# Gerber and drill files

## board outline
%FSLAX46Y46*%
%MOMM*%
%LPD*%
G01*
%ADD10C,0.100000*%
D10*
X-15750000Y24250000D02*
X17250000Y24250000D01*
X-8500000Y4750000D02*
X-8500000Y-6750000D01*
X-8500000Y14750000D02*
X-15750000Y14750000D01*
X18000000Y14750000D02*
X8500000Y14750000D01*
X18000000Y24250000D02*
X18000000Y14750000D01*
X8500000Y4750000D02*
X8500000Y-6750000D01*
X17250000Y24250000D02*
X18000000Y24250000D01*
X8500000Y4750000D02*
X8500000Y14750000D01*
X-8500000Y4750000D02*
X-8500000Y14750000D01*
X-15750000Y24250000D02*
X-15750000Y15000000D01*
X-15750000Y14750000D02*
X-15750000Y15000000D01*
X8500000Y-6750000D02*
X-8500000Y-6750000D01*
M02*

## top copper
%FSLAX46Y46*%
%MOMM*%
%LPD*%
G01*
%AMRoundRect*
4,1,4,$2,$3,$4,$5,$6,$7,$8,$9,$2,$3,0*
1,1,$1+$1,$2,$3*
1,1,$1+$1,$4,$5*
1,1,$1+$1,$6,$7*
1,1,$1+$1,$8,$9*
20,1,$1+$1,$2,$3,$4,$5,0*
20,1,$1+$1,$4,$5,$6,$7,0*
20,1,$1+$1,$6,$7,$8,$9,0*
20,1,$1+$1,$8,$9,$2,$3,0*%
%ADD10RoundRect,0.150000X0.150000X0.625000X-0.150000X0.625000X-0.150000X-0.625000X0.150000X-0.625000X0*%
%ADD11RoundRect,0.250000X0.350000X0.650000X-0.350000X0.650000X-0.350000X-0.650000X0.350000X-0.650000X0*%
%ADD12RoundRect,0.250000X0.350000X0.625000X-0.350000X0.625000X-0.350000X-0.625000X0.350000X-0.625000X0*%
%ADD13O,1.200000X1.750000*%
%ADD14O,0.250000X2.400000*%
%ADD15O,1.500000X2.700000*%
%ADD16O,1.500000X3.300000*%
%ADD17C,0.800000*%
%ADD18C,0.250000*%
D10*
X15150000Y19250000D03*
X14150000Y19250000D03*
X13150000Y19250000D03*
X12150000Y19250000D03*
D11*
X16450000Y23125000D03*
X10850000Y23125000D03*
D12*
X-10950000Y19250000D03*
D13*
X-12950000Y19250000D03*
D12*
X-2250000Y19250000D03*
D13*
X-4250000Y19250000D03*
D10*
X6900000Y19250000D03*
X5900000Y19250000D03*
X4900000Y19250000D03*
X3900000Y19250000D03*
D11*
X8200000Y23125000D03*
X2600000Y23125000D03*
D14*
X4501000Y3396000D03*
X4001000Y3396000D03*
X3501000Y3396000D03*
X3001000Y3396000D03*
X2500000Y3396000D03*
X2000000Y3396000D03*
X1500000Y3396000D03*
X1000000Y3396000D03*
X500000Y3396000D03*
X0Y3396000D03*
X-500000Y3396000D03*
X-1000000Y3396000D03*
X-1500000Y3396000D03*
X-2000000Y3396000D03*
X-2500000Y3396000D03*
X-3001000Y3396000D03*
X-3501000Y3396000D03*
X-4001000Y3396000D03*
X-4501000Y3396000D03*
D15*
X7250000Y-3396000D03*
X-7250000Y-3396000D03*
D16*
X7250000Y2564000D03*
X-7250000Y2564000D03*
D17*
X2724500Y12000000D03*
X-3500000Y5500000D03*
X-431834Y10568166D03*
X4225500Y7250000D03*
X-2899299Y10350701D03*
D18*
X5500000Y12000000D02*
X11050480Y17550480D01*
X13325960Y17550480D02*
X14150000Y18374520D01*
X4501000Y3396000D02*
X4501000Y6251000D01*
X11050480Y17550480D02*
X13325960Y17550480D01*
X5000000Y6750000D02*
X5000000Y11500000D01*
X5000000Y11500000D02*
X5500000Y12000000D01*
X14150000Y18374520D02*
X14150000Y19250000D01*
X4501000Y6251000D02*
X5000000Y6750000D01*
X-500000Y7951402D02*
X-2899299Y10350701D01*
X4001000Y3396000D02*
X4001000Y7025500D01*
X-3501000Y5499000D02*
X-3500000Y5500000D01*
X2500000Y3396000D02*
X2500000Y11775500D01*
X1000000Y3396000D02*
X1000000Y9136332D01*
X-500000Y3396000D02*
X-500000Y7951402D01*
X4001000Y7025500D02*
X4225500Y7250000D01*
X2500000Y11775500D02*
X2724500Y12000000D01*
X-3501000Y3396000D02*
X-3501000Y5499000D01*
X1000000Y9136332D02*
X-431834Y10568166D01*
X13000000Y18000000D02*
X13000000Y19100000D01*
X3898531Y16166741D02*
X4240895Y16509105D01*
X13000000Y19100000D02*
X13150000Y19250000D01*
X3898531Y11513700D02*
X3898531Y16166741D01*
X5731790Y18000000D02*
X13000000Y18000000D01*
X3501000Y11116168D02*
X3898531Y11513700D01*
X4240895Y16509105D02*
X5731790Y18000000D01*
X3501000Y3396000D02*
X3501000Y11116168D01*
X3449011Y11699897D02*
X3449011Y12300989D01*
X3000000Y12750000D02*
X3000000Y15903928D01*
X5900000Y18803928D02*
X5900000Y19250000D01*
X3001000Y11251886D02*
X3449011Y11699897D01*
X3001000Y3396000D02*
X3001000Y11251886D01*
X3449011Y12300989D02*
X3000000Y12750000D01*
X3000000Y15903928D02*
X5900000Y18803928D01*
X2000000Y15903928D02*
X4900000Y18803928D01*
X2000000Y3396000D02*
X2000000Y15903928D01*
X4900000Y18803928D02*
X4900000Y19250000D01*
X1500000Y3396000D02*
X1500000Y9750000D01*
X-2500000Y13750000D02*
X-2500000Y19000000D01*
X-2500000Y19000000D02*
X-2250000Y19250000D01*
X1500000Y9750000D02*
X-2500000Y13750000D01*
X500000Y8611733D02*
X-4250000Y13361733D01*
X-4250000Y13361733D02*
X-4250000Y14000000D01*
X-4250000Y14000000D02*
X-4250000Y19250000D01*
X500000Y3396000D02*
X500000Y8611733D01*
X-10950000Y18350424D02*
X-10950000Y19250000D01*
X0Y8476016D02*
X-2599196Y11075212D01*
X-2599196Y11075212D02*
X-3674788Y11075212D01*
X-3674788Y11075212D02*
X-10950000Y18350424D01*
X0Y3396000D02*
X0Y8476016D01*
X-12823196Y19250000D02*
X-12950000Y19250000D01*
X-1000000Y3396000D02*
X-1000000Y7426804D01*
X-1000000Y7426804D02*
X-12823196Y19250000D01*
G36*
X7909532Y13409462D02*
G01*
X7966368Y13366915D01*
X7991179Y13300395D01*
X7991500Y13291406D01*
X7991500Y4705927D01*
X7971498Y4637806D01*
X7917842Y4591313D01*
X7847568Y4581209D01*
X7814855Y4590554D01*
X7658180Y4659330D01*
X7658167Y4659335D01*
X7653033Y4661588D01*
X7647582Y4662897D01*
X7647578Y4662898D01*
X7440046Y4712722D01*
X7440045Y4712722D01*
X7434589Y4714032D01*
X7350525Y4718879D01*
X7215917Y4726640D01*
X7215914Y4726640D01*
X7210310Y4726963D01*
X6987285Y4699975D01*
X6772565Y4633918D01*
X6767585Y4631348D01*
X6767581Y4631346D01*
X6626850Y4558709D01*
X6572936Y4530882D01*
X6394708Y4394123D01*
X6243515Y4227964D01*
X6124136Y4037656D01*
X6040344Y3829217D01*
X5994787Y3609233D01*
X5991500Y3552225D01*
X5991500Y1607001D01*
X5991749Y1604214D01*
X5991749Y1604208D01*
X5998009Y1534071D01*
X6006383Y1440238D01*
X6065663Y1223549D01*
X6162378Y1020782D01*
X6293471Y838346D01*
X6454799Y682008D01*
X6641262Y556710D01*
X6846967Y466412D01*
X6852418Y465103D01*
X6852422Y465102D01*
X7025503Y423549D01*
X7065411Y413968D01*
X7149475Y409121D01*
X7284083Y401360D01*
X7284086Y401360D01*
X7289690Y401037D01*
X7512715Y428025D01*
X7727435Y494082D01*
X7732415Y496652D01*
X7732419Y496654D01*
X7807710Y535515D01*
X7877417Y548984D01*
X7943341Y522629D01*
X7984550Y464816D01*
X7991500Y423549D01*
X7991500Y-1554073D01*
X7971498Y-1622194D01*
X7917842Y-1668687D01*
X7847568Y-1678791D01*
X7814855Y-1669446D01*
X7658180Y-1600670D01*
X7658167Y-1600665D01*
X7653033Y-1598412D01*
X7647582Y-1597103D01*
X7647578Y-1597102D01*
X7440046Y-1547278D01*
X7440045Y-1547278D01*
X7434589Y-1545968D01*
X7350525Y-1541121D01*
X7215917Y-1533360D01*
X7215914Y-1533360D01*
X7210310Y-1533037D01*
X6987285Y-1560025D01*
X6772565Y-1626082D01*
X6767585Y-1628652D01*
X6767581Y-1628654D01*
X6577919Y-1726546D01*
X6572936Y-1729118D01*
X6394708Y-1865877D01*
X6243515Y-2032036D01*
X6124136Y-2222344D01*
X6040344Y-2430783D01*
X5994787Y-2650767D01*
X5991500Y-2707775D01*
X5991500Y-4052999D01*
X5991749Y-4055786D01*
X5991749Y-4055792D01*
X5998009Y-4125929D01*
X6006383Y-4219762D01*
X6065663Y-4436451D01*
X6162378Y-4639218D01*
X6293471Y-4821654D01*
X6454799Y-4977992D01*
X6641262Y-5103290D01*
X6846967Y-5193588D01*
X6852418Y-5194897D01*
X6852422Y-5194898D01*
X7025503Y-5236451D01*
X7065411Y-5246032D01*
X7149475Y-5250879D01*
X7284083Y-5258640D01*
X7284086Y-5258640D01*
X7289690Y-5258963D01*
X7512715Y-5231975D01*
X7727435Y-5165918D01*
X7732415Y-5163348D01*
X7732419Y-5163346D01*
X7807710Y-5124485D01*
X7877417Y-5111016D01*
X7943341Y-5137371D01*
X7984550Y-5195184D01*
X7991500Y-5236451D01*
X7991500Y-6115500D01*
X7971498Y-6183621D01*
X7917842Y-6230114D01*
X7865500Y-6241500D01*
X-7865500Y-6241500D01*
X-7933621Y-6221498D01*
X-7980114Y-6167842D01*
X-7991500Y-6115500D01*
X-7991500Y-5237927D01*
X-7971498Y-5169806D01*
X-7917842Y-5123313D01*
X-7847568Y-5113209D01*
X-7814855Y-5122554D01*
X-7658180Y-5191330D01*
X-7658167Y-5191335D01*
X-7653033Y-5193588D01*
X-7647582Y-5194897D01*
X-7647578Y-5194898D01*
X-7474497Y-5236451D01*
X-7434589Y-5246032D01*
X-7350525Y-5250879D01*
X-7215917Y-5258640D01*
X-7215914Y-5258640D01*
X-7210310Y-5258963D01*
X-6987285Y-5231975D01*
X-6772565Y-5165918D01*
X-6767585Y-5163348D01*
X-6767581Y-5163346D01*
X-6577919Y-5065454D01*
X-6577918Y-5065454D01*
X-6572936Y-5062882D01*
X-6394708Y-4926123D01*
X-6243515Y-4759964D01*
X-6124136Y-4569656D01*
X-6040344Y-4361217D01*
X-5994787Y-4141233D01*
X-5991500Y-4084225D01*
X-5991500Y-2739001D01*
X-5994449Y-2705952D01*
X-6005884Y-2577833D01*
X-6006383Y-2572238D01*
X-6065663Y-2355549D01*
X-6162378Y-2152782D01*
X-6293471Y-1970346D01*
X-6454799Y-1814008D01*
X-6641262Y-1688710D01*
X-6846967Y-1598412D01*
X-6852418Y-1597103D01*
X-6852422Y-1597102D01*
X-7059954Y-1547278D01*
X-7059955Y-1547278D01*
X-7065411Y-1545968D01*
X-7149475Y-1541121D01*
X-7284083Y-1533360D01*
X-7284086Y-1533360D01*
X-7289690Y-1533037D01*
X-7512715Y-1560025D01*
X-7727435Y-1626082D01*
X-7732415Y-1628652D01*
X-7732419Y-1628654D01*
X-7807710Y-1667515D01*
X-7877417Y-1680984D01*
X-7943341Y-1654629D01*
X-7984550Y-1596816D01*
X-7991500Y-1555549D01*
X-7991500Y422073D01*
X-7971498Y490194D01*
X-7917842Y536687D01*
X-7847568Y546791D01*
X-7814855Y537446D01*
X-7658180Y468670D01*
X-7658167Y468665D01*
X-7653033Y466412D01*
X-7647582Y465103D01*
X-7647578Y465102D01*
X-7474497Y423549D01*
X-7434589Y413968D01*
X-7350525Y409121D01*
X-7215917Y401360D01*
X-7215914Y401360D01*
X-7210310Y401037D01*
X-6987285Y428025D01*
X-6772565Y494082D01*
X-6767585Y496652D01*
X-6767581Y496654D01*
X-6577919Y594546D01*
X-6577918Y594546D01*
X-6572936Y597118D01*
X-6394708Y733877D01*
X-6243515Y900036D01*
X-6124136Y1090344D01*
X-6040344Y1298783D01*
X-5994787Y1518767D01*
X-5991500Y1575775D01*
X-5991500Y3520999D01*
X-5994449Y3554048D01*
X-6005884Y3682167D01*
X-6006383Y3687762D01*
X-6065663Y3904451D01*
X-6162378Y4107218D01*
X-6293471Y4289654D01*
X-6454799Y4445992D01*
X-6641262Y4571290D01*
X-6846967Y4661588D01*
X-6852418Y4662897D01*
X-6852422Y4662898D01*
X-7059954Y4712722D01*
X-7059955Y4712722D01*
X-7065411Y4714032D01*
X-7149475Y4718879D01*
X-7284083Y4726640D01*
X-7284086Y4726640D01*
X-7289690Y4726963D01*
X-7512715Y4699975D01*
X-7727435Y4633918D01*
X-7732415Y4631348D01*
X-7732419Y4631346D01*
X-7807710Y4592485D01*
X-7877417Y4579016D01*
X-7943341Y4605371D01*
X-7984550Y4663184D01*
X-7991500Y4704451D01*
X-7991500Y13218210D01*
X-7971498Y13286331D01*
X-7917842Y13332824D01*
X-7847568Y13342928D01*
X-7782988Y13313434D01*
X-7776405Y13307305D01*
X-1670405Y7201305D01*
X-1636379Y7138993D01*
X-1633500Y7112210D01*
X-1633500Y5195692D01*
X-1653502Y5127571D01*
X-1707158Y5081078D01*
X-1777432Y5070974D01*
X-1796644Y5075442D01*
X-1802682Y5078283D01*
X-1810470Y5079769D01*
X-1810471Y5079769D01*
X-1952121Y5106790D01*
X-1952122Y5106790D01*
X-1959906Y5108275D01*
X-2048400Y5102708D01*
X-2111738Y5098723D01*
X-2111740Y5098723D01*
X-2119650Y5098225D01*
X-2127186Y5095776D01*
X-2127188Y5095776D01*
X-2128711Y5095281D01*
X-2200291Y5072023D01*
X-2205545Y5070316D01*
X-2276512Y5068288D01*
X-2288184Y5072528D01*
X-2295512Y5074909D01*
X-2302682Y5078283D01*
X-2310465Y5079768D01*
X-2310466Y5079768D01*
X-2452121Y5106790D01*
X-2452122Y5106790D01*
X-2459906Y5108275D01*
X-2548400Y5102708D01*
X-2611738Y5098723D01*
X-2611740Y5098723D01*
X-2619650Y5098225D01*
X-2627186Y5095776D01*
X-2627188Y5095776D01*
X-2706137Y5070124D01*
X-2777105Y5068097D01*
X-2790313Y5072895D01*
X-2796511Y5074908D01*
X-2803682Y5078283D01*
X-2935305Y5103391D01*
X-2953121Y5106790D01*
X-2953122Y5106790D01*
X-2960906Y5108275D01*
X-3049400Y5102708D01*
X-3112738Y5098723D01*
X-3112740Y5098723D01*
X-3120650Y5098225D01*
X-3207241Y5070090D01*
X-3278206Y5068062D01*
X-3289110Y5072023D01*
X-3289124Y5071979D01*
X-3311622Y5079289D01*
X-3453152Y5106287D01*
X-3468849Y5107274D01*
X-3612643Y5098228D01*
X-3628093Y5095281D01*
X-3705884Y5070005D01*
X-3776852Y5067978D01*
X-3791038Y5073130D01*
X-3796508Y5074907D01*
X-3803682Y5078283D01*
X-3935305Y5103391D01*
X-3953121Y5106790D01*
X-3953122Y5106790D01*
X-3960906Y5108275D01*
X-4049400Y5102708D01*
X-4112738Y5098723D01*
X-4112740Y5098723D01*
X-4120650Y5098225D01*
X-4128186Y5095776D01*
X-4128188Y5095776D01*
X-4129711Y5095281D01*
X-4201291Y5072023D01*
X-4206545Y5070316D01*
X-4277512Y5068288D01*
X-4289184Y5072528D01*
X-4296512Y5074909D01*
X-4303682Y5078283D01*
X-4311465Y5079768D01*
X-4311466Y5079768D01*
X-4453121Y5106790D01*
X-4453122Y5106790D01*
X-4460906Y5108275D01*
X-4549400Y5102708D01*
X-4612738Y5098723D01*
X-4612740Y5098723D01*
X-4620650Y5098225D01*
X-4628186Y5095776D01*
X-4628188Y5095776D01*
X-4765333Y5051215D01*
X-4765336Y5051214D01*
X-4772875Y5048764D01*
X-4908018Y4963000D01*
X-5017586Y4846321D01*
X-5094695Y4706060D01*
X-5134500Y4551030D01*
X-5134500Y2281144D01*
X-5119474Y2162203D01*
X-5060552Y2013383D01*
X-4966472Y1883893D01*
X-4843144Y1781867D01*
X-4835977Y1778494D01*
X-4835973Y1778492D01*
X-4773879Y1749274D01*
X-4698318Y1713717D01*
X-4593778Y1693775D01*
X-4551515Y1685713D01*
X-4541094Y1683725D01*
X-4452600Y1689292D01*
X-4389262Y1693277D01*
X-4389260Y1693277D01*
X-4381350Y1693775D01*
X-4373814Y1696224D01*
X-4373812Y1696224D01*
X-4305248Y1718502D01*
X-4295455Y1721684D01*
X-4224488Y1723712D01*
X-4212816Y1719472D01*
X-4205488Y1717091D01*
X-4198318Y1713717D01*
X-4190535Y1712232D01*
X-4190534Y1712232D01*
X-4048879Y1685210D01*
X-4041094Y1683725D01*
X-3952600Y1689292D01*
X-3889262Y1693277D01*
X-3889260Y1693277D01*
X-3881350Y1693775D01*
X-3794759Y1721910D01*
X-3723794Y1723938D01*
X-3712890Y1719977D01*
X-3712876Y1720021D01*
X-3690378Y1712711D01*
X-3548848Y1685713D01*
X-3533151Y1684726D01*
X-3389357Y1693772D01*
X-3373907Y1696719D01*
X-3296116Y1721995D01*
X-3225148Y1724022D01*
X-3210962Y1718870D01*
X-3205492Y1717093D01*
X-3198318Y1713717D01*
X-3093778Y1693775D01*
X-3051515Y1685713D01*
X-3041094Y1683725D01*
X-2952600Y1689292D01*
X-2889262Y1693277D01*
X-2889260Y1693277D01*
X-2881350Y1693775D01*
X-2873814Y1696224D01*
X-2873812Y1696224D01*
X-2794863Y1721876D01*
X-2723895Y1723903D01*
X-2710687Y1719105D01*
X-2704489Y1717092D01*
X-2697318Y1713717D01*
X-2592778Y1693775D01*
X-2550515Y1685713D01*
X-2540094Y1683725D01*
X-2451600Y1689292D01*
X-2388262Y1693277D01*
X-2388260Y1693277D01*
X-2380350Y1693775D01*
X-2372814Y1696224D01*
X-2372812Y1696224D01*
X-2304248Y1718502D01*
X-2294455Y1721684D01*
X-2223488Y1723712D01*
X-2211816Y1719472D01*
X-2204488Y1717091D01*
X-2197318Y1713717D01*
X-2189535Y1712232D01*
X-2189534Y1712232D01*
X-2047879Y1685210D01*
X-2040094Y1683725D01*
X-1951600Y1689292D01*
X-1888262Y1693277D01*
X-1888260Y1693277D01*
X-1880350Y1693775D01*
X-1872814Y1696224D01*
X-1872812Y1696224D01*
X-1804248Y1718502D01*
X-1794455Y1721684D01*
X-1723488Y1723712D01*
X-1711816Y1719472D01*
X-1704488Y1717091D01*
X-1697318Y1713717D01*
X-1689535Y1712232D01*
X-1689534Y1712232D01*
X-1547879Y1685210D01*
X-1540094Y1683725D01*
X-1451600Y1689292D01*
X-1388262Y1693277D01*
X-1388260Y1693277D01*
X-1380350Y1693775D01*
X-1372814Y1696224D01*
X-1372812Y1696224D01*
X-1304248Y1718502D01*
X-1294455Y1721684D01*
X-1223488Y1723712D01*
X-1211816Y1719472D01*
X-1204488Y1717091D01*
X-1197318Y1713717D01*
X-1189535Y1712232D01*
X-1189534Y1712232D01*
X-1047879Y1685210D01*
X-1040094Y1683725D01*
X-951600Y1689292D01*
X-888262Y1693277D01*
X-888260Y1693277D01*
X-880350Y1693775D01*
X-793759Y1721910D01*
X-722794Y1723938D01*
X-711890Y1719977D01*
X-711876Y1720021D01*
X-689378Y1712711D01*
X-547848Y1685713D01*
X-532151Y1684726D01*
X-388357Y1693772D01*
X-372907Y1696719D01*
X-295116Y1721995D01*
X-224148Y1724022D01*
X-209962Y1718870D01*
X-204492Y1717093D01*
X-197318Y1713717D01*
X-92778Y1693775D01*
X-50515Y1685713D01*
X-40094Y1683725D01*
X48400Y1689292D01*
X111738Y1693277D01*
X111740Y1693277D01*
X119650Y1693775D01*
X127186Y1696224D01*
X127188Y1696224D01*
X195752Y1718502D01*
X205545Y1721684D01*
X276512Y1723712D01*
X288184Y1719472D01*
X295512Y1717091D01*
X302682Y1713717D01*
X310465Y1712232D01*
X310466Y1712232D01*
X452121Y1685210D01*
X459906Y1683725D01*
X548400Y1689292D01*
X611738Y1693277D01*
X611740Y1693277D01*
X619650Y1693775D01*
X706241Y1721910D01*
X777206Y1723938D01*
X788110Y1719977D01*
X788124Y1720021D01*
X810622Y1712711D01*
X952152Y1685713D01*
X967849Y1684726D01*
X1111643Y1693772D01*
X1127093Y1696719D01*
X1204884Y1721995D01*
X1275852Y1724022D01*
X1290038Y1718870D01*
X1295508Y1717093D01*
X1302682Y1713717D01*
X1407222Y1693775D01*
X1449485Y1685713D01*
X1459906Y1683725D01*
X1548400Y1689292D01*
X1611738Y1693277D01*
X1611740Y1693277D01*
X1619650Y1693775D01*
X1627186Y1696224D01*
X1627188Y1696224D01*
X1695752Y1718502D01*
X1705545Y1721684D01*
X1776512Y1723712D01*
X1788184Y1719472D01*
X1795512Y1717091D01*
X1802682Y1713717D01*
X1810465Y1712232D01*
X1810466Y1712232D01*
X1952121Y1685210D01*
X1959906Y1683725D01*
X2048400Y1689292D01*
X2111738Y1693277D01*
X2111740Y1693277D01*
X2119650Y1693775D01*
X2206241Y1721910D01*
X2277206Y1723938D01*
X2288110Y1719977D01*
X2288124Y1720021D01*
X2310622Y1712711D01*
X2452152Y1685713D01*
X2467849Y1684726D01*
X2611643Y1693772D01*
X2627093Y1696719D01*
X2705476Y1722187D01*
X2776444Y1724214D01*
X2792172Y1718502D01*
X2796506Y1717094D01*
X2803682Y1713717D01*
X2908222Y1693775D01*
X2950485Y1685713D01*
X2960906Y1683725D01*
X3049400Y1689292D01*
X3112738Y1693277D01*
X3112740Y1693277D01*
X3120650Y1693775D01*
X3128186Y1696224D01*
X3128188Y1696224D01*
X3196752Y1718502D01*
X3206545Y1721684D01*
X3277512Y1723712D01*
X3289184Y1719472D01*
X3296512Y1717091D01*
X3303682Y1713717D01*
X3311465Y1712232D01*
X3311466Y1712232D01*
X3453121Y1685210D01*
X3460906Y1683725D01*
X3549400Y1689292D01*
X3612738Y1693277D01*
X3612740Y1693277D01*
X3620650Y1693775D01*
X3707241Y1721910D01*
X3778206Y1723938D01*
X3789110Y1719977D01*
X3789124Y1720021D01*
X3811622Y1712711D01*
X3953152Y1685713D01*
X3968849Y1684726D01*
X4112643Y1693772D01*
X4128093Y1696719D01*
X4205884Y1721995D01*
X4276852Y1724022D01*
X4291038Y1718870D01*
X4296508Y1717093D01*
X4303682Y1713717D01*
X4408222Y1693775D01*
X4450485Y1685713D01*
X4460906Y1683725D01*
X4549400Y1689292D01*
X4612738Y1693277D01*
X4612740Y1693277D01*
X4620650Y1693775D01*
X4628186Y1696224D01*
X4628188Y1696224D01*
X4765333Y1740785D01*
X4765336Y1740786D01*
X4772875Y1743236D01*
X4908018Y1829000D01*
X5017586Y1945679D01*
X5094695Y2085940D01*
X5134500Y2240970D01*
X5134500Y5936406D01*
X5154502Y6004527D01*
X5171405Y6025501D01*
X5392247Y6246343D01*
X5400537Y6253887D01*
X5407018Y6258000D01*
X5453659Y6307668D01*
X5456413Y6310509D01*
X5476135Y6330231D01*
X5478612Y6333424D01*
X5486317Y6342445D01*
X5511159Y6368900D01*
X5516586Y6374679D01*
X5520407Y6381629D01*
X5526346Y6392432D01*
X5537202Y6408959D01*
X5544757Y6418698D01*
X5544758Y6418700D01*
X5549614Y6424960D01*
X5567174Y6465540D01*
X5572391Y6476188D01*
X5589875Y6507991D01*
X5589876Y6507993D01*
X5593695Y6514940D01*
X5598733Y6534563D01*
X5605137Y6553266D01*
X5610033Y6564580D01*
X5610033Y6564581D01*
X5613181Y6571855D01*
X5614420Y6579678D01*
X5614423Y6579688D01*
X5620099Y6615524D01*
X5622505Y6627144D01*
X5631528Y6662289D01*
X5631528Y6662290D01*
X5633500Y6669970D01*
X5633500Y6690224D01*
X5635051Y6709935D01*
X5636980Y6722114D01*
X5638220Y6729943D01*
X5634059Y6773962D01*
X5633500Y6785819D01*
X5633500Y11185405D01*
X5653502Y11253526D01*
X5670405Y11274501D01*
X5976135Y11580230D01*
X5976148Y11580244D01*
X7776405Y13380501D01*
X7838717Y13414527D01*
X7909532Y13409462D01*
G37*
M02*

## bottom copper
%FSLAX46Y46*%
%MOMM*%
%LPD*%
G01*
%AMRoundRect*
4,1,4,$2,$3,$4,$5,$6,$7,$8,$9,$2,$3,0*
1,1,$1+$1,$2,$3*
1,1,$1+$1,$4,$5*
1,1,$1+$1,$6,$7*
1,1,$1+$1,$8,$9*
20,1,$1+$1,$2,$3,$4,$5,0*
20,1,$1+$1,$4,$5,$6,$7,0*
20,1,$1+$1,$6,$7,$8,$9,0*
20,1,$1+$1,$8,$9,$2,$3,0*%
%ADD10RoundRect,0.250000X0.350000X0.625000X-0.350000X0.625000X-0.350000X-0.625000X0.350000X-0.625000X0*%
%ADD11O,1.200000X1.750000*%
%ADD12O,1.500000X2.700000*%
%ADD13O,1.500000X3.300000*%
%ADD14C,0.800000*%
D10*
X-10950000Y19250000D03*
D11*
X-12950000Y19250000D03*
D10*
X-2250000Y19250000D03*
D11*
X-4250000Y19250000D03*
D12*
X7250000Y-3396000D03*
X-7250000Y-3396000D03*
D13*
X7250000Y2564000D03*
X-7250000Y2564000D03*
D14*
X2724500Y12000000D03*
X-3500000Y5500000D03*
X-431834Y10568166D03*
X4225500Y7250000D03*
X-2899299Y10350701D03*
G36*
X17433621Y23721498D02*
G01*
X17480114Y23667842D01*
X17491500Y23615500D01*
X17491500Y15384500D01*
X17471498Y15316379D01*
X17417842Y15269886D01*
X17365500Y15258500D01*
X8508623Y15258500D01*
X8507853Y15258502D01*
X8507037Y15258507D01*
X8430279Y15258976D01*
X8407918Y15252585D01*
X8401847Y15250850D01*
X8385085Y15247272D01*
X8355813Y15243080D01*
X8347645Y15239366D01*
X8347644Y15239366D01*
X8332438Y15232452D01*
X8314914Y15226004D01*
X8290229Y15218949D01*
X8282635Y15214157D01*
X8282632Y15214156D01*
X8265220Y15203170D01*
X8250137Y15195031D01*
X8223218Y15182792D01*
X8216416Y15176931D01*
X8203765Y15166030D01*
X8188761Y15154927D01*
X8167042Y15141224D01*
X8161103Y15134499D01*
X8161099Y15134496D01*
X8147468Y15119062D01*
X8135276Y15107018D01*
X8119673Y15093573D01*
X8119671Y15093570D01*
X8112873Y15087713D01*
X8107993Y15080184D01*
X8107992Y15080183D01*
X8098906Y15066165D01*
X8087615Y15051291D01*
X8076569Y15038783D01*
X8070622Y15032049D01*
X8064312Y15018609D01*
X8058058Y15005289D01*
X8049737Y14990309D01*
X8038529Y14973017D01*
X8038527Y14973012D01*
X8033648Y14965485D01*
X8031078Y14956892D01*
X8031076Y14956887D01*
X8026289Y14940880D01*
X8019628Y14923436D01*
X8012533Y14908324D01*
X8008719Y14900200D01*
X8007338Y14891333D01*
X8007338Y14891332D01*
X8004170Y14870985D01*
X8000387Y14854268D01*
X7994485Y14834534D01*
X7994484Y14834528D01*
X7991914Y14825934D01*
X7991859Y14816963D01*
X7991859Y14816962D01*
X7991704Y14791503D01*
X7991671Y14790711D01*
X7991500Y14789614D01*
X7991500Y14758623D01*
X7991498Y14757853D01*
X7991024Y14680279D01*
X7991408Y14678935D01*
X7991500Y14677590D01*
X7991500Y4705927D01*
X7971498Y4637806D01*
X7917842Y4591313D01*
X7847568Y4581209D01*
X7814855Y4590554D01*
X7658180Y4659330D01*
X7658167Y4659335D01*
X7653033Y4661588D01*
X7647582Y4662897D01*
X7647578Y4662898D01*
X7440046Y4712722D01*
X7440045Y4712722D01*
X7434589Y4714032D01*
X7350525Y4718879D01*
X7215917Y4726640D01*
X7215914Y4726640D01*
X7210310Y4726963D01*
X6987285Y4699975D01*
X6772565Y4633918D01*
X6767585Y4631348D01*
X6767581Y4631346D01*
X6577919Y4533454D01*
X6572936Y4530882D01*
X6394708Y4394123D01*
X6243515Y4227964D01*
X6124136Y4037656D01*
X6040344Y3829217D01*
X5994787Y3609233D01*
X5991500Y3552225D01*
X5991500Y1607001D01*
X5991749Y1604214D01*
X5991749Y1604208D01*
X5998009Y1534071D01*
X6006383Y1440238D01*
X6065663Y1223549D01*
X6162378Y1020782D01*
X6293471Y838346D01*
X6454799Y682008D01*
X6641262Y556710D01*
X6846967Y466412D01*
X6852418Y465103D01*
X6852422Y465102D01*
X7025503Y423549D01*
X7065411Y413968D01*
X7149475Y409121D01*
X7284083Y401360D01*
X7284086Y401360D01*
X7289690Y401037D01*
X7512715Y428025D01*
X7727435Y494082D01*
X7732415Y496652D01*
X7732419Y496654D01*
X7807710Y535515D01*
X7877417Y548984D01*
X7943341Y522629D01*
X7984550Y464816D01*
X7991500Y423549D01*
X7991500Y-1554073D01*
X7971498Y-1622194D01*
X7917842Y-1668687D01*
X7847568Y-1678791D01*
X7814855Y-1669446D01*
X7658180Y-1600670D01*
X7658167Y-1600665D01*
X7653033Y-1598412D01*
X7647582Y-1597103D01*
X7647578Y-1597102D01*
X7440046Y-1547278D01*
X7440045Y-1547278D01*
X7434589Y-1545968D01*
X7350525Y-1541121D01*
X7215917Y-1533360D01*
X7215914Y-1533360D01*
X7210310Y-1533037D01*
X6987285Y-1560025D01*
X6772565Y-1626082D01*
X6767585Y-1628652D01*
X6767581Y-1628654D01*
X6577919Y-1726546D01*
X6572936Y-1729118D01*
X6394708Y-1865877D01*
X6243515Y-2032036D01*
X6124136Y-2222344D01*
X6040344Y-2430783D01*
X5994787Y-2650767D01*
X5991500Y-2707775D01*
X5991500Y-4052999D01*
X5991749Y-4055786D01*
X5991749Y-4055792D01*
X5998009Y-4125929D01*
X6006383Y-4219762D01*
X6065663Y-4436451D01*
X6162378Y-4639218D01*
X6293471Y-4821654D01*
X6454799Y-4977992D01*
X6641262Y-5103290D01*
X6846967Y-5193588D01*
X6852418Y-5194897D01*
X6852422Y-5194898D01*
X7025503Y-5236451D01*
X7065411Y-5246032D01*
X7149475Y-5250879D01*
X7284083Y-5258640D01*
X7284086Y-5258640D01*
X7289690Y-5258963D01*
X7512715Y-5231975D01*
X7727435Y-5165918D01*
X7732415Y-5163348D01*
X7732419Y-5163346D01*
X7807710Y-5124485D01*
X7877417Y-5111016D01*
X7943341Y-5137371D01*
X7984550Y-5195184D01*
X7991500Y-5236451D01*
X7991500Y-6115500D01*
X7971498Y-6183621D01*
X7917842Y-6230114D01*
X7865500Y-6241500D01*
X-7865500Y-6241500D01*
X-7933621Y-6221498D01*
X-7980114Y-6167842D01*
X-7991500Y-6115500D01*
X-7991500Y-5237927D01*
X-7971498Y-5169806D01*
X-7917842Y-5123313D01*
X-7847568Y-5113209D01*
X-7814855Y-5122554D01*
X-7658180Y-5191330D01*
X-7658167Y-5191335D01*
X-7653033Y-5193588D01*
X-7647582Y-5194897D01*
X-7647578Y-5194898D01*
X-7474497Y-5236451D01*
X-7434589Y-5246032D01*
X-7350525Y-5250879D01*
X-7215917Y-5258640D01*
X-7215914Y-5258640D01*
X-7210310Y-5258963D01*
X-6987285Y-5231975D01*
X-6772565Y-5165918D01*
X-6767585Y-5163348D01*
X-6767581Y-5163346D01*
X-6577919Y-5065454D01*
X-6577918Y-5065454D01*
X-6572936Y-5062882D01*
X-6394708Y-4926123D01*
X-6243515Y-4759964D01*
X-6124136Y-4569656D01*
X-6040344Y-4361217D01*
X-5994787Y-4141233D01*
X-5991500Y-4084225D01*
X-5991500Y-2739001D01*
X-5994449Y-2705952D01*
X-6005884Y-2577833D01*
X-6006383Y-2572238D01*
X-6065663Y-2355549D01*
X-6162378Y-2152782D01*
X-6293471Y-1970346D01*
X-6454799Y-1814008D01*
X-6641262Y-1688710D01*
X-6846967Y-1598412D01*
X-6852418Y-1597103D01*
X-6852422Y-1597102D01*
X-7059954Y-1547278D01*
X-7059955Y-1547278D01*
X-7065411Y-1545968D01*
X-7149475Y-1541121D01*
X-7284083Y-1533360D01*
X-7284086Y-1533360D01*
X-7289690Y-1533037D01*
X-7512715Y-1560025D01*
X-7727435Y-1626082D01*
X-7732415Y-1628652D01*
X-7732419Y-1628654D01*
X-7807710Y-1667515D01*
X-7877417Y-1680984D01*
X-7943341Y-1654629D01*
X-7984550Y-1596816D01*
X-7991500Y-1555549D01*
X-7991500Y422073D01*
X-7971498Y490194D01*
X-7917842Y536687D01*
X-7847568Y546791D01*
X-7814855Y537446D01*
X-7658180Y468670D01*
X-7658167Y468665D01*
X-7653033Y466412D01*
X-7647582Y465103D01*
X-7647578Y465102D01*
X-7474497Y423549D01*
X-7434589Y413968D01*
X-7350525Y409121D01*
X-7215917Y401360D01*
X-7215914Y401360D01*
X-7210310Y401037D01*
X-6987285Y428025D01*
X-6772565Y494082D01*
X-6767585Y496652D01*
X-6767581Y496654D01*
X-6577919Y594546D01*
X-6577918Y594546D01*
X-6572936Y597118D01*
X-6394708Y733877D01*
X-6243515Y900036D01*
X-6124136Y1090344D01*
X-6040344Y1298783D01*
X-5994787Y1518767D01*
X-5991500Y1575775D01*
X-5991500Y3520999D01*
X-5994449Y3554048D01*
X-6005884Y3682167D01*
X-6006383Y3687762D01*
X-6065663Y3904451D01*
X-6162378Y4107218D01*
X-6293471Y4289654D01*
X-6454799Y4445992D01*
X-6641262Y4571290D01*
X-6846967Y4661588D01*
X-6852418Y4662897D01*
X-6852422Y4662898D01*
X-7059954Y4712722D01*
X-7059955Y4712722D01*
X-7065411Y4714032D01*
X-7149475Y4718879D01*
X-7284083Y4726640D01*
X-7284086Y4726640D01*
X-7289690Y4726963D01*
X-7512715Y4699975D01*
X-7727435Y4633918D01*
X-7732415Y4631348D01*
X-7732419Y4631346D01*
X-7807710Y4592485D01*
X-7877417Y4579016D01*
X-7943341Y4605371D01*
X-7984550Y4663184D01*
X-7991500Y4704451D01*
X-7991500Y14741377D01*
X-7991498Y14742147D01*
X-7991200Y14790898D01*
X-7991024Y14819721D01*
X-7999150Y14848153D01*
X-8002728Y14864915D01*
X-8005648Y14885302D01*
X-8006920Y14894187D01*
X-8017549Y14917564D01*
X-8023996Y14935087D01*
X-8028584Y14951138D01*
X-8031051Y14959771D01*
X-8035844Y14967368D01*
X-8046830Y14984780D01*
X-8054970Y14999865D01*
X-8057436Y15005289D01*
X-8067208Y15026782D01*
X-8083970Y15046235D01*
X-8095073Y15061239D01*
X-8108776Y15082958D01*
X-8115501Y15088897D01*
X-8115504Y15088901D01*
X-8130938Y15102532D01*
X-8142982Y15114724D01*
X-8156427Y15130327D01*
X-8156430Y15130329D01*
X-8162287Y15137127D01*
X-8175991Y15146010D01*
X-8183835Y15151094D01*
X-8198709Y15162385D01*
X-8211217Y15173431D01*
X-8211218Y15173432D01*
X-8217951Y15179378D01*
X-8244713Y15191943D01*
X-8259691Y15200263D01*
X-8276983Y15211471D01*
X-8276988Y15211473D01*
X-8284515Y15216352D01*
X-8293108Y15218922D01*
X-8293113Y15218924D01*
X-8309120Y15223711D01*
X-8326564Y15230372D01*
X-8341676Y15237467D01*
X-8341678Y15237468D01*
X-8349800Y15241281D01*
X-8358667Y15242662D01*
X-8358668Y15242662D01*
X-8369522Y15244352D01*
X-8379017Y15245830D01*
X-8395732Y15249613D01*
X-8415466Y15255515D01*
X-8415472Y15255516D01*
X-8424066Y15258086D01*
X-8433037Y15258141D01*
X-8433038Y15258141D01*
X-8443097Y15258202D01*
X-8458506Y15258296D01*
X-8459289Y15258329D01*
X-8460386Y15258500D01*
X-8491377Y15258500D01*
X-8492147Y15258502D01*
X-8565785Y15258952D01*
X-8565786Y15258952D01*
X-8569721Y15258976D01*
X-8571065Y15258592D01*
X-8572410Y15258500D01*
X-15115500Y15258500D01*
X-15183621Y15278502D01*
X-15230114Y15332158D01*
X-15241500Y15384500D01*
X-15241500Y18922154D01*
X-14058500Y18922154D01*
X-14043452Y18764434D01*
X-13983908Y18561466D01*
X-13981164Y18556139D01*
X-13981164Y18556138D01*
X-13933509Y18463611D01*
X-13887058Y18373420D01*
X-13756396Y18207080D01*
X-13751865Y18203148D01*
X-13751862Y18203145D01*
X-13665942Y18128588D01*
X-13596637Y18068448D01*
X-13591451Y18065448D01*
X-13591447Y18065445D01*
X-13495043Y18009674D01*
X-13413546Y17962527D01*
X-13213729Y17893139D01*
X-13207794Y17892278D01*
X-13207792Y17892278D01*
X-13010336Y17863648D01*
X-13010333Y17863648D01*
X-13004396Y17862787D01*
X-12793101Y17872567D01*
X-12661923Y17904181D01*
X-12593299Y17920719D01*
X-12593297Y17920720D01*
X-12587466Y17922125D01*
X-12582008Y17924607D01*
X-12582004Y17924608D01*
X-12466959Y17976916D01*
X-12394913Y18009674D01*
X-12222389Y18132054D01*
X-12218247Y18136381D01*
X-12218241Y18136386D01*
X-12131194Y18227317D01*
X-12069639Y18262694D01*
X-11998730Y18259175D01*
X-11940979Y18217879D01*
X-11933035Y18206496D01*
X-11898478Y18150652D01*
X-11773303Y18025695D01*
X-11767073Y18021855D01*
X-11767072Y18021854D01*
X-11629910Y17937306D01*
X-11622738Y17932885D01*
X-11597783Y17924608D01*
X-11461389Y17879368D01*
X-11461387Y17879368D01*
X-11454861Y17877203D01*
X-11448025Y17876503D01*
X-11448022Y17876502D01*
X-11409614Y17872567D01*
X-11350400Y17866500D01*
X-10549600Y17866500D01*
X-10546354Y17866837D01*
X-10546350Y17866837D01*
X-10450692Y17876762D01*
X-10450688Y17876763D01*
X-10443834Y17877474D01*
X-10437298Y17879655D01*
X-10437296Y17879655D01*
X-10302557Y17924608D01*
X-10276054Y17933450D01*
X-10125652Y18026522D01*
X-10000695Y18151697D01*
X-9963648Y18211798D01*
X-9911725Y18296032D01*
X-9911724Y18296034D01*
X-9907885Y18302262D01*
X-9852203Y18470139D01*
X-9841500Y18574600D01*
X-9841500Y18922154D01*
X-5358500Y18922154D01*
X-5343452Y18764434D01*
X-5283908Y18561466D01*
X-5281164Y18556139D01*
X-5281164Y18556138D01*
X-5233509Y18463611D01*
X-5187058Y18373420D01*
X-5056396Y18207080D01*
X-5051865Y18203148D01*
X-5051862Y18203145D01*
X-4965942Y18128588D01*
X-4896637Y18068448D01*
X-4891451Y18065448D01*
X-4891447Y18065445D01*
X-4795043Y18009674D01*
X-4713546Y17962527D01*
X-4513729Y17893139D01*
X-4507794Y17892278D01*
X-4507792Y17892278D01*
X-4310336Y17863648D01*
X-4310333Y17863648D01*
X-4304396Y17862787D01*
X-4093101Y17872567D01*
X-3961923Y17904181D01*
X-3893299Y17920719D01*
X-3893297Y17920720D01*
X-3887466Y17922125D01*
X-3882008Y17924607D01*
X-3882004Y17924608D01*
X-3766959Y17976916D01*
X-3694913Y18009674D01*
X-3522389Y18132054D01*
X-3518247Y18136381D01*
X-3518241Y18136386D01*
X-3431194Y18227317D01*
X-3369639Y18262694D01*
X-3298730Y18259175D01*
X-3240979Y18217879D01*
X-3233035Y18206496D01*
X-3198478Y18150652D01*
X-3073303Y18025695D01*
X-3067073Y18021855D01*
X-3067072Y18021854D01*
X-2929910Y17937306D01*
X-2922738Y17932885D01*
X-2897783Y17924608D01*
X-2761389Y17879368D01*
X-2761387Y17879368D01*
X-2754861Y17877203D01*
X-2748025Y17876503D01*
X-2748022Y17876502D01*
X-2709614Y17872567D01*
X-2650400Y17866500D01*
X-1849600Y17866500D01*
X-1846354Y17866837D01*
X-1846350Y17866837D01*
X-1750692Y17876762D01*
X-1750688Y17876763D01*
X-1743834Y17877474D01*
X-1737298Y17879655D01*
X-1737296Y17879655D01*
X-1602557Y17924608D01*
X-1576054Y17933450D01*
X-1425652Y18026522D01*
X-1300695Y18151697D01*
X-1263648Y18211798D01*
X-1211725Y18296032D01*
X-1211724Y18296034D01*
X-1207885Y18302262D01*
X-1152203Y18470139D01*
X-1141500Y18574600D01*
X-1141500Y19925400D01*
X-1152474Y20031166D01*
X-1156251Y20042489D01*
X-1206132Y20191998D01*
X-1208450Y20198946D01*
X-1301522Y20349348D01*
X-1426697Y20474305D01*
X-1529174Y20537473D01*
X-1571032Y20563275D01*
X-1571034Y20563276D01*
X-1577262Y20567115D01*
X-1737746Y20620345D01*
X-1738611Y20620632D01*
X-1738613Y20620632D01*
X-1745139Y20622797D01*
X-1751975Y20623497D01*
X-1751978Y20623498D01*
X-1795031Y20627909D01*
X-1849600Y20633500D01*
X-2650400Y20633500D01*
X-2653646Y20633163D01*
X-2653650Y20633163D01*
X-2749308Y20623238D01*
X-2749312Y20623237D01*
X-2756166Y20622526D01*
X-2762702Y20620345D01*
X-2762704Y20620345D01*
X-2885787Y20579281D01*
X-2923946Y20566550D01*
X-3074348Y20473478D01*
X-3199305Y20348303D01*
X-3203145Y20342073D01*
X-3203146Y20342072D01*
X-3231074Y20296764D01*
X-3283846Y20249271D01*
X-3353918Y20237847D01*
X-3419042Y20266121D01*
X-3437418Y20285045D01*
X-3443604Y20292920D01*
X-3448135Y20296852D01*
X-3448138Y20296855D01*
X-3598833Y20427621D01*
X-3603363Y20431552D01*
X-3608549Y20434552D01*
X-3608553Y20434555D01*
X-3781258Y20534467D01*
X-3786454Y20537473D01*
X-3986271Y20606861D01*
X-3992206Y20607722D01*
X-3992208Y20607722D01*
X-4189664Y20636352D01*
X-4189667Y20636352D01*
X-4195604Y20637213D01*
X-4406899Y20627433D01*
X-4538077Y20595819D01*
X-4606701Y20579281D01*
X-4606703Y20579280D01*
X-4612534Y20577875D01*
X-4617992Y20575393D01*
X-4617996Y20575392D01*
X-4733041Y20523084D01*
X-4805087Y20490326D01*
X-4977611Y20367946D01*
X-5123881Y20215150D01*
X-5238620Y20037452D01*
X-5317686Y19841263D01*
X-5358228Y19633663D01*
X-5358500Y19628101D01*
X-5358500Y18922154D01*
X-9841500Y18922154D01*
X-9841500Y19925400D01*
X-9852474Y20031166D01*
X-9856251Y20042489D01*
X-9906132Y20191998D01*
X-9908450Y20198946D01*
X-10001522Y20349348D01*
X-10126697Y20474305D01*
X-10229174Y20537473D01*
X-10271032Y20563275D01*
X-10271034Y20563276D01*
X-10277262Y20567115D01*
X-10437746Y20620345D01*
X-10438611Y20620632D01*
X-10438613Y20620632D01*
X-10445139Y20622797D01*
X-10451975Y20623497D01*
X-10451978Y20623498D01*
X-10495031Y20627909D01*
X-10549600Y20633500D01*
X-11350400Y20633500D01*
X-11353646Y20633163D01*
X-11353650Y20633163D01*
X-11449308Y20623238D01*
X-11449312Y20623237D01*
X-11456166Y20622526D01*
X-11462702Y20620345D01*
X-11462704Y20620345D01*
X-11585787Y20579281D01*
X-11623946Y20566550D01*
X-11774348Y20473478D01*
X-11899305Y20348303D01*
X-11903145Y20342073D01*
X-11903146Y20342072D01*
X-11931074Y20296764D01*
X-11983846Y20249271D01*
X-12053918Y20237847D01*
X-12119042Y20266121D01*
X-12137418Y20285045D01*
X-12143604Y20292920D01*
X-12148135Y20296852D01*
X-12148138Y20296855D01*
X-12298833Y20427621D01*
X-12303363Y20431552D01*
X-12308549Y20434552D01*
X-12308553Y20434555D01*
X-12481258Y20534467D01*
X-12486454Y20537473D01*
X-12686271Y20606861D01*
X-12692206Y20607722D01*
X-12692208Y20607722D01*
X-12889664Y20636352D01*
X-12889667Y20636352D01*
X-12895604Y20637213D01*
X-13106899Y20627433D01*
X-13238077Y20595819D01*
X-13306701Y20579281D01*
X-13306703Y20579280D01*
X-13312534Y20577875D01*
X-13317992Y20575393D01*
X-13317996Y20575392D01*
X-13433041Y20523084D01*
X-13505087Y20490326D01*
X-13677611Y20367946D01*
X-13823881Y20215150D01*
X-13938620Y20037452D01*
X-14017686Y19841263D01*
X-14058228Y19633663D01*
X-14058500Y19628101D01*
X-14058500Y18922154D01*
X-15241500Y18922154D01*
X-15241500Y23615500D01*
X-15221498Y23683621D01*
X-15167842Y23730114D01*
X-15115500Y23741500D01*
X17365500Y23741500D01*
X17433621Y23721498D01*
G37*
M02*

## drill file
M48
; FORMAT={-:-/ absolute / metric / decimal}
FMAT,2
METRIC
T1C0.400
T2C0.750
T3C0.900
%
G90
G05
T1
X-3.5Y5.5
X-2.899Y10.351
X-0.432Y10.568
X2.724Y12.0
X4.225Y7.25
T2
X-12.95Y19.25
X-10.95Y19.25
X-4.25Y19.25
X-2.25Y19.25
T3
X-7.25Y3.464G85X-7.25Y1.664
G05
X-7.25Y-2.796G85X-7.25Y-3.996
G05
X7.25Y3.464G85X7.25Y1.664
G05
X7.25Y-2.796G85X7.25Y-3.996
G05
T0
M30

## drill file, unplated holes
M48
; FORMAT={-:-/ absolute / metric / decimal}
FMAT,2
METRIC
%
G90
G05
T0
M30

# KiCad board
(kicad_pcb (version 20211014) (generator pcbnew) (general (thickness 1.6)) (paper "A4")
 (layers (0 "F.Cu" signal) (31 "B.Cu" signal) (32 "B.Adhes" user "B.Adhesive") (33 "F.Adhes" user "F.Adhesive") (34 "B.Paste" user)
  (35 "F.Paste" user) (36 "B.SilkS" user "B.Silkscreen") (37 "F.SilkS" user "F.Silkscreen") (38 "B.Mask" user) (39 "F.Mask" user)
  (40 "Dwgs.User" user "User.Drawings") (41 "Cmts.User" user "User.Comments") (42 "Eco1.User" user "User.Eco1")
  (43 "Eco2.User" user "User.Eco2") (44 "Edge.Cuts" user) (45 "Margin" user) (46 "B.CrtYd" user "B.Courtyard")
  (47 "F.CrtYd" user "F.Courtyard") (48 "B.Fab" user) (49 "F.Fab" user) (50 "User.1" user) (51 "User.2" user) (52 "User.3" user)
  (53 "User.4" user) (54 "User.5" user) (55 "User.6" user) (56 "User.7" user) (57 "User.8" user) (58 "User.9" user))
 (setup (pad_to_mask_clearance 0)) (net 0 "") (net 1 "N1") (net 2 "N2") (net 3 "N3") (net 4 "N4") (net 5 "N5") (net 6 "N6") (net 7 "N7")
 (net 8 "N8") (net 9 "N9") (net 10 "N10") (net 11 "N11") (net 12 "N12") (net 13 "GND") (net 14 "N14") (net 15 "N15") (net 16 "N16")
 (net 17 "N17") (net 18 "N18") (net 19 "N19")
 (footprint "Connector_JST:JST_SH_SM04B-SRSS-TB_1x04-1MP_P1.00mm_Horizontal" (layer "F.Cu") (at 13.65 -21.25 180)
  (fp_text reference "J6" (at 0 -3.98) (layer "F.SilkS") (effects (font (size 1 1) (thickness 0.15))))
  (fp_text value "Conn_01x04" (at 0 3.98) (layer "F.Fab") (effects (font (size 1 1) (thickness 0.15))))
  (pad "1" smd roundrect (at -1.5 -2 180) (size 0.6 1.55) (layers "F.Cu" "F.Paste" "F.Mask") (roundrect_rratio 0.25) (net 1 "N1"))
  (pad "2" smd roundrect (at -0.5 -2 180) (size 0.6 1.55) (layers "F.Cu" "F.Paste" "F.Mask") (roundrect_rratio 0.25) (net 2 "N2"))
  (pad "3" smd roundrect (at 0.5 -2 180) (size 0.6 1.55) (layers "F.Cu" "F.Paste" "F.Mask") (roundrect_rratio 0.25) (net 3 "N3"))
  (pad "4" smd roundrect (at 1.5 -2 180) (size 0.6 1.55) (layers "F.Cu" "F.Paste" "F.Mask") (roundrect_rratio 0.25) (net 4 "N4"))
  (pad "MP" smd roundrect (at -2.8 1.875 180) (size 1.2 1.8) (layers "F.Cu" "F.Paste" "F.Mask") (roundrect_rratio 0.2083333333))
  (pad "MP" smd roundrect (at 2.8 1.875 180) (size 1.2 1.8) (layers "F.Cu" "F.Paste" "F.Mask") (roundrect_rratio 0.2083333333)))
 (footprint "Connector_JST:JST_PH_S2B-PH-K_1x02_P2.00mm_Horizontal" (layer "F.Cu") (at -10.95 -19.25 180)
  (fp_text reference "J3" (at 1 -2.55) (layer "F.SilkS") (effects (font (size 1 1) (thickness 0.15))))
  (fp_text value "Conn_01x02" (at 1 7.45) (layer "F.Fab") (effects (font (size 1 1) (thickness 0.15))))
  (pad "1" thru_hole roundrect (at 0 0 180) (size 1.2 1.75) (drill 0.75) (layers *.Cu *.Mask) (roundrect_rratio 0.2083333333) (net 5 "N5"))
  (pad "2" thru_hole oval (at 2 0 180) (size 1.2 1.75) (drill 0.75) (layers *.Cu *.Mask) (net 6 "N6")))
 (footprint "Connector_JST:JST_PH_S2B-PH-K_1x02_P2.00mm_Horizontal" (layer "F.Cu") (at -2.25 -19.25 180)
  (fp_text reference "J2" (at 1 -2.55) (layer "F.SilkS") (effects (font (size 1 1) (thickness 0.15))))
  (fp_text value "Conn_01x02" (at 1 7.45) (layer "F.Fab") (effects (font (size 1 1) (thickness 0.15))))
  (pad "1" thru_hole roundrect (at 0 0 180) (size 1.2 1.75) (drill 0.75) (layers *.Cu *.Mask) (roundrect_rratio 0.2083333333) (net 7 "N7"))
  (pad "2" thru_hole oval (at 2 0 180) (size 1.2 1.75) (drill 0.75) (layers *.Cu *.Mask) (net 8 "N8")))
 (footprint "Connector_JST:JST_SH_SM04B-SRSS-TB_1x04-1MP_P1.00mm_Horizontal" (layer "F.Cu") (at 5.4 -21.25 180)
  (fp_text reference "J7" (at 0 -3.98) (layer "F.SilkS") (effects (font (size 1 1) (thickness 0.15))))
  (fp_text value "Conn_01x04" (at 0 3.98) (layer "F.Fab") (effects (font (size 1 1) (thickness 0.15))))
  (pad "1" smd roundrect (at -1.5 -2 180) (size 0.6 1.55) (layers "F.Cu" "F.Paste" "F.Mask") (roundrect_rratio 0.25) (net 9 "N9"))
  (pad "2" smd roundrect (at -0.5 -2 180) (size 0.6 1.55) (layers "F.Cu" "F.Paste" "F.Mask") (roundrect_rratio 0.25) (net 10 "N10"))
  (pad "3" smd roundrect (at 0.5 -2 180) (size 0.6 1.55) (layers "F.Cu" "F.Paste" "F.Mask") (roundrect_rratio 0.25) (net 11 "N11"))
  (pad "4" smd roundrect (at 1.5 -2 180) (size 0.6 1.55) (layers "F.Cu" "F.Paste" "F.Mask") (roundrect_rratio 0.25) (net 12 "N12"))
  (pad "MP" smd roundrect (at -2.8 1.875 180) (size 1.2 1.8) (layers "F.Cu" "F.Paste" "F.Mask") (roundrect_rratio 0.2083333333))
  (pad "MP" smd roundrect (at 2.8 1.875 180) (size 1.2 1.8) (layers "F.Cu" "F.Paste" "F.Mask") (roundrect_rratio 0.2083333333)))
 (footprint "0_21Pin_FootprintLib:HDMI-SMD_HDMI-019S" (layer "F.Cu") (at 0 0)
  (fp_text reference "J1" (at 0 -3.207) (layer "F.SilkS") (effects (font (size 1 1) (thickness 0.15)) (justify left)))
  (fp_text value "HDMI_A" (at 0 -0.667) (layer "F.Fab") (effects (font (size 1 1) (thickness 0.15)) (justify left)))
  (pad "1" smd oval (at 4.501 -3.396) (size 0.25 2.4) (layers "F.Cu" "F.Paste" "F.Mask") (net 2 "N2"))
  (pad "2" smd oval (at 4.001 -3.396) (size 0.25 2.4) (layers "F.Cu" "F.Paste" "F.Mask") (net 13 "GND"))
  (pad "3" smd oval (at 3.501 -3.396) (size 0.25 2.4) (layers "F.Cu" "F.Paste" "F.Mask") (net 3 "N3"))
  (pad "4" smd oval (at 3.001 -3.396) (size 0.25 2.4) (layers "F.Cu" "F.Paste" "F.Mask") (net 10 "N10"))
  (pad "5" smd oval (at 2.5 -3.396) (size 0.25 2.4) (layers "F.Cu" "F.Paste" "F.Mask") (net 13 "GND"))
  (pad "6" smd oval (at 2 -3.396) (size 0.25 2.4) (layers "F.Cu" "F.Paste" "F.Mask") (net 11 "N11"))
  (pad "7" smd oval (at 1.5 -3.396) (size 0.25 2.4) (layers "F.Cu" "F.Paste" "F.Mask") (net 7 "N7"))
  (pad "8" smd oval (at 1 -3.396) (size 0.25 2.4) (layers "F.Cu" "F.Paste" "F.Mask") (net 13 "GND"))
  (pad "9" smd oval (at 0.5 -3.396) (size 0.25 2.4) (layers "F.Cu" "F.Paste" "F.Mask") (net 8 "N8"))
  (pad "10" smd oval (at 0 -3.396) (size 0.25 2.4) (layers "F.Cu" "F.Paste" "F.Mask") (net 5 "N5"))
  (pad "11" smd oval (at -0.5 -3.396) (size 0.25 2.4) (layers "F.Cu" "F.Paste" "F.Mask") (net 13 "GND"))
  (pad "12" smd oval (at -1 -3.396) (size 0.25 2.4) (layers "F.Cu" "F.Paste" "F.Mask") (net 6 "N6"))
  (pad "13" smd oval (at -1.5 -3.396) (size 0.25 2.4) (layers "F.Cu" "F.Paste" "F.Mask") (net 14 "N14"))
  (pad "14" smd oval (at -2 -3.396) (size 0.25 2.4) (layers "F.Cu" "F.Paste" "F.Mask") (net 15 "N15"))
  (pad "15" smd oval (at -2.5 -3.396) (size 0.25 2.4) (layers "F.Cu" "F.Paste" "F.Mask") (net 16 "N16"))
  (pad "16" smd oval (at -3.001 -3.396) (size 0.25 2.4) (layers "F.Cu" "F.Paste" "F.Mask") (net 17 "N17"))
  (pad "17" smd oval (at -3.501 -3.396) (size 0.25 2.4) (layers "F.Cu" "F.Paste" "F.Mask") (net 13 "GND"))
  (pad "18" smd oval (at -4.001 -3.396) (size 0.25 2.4) (layers "F.Cu" "F.Paste" "F.Mask") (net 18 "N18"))
  (pad "19" smd oval (at -4.501 -3.396) (size 0.25 2.4) (layers "F.Cu" "F.Paste" "F.Mask") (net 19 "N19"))
  (pad "20" thru_hole oval (at 7.25 3.396) (size 1.5 2.7) (drill oval 0.9 2.1) (layers *.Cu *.Mask))
  (pad "21" thru_hole oval (at -7.25 3.396) (size 1.5 2.7) (drill oval 0.9 2.1) (layers *.Cu *.Mask))
  (pad "22" thru_hole oval (at 7.25 -2.564) (size 1.5 3.3) (drill oval 0.9 2.7) (layers *.Cu *.Mask))
  (pad "23" thru_hole oval (at -7.25 -2.564) (size 1.5 3.3) (drill oval 0.9 2.7) (layers *.Cu *.Mask)))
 (gr_line (start -15.75 -24.25) (end 17.25 -24.25) (layer "Edge.Cuts") (width 0.1))
 (gr_line (start -8.5 -4.75) (end -8.5 6.75) (layer "Edge.Cuts") (width 0.1))
 (gr_line (start -8.5 -14.75) (end -15.75 -14.75) (layer "Edge.Cuts") (width 0.1))
 (gr_line (start 18 -14.75) (end 8.5 -14.75) (layer "Edge.Cuts") (width 0.1))
 (gr_line (start 18 -24.25) (end 18 -14.75) (layer "Edge.Cuts") (width 0.1))
 (gr_line (start 8.5 -4.75) (end 8.5 6.75) (layer "Edge.Cuts") (width 0.1))
 (gr_line (start 17.25 -24.25) (end 18 -24.25) (layer "Edge.Cuts") (width 0.1))
 (gr_line (start 8.5 -4.75) (end 8.5 -14.75) (layer "Edge.Cuts") (width 0.1))
 (gr_line (start -8.5 -4.75) (end -8.5 -14.75) (layer "Edge.Cuts") (width 0.1))
 (gr_line (start -15.75 -24.25) (end -15.75 -15) (layer "Edge.Cuts") (width 0.1))
 (gr_line (start -15.75 -14.75) (end -15.75 -15) (layer "Edge.Cuts") (width 0.1))
 (gr_line (start 8.5 6.75) (end -8.5 6.75) (layer "Edge.Cuts") (width 0.1))
 (segment (start 5.5 -12) (end 11.05048 -17.55048) (width 0.25) (layer "F.Cu") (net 2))
 (segment (start 13.32596 -17.55048) (end 14.15 -18.37452) (width 0.25) (layer "F.Cu") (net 2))
 (segment (start 4.501 -3.396) (end 4.501 -6.251) (width 0.25) (layer "F.Cu") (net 2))
 (segment (start 11.05048 -17.55048) (end 13.32596 -17.55048) (width 0.25) (layer "F.Cu") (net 2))
 (segment (start 5 -6.75) (end 5 -11.5) (width 0.25) (layer "F.Cu") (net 2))
 (segment (start 5 -11.5) (end 5.5 -12) (width 0.25) (layer "F.Cu") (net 2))
 (segment (start 14.15 -18.37452) (end 14.15 -19.25) (width 0.25) (layer "F.Cu") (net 2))
 (segment (start 4.501 -6.251) (end 5 -6.75) (width 0.25) (layer "F.Cu") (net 2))
 (segment (start -0.5 -7.951402) (end -2.899299 -10.350701) (width 0.25) (layer "F.Cu") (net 13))
 (segment (start 4.001 -3.396) (end 4.001 -7.0255) (width 0.25) (layer "F.Cu") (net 13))
 (segment (start -3.501 -5.499) (end -3.5 -5.5) (width 0.25) (layer "F.Cu") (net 13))
 (segment (start 2.5 -3.396) (end 2.5 -11.7755) (width 0.25) (layer "F.Cu") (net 13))
 (segment (start 1 -3.396) (end 1 -9.136332) (width 0.25) (layer "F.Cu") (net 13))
 (segment (start -0.5 -3.396) (end -0.5 -7.951402) (width 0.25) (layer "F.Cu") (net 13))
 (segment (start 4.001 -7.0255) (end 4.2255 -7.25) (width 0.25) (layer "F.Cu") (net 13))
 (segment (start 2.5 -11.7755) (end 2.7245 -12) (width 0.25) (layer "F.Cu") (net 13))
 (segment (start -3.501 -3.396) (end -3.501 -5.499) (width 0.25) (layer "F.Cu") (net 13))
 (segment (start 1 -9.136332) (end -0.431834 -10.568166) (width 0.25) (layer "F.Cu") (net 13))
 (via (at 2.7245 -12) (size 0.8) (drill 0.4) (layers "F.Cu" "B.Cu") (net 13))
 (via (at -3.5 -5.5) (size 0.8) (drill 0.4) (layers "F.Cu" "B.Cu") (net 13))
 (via (at -0.431834 -10.568166) (size 0.8) (drill 0.4) (layers "F.Cu" "B.Cu") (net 13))
 (via (at 4.2255 -7.25) (size 0.8) (drill 0.4) (layers "F.Cu" "B.Cu") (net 13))
 (via (at -2.899299 -10.350701) (size 0.8) (drill 0.4) (layers "F.Cu" "B.Cu") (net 13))
 (segment (start 13 -18) (end 13 -19.1) (width 0.25) (layer "F.Cu") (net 3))
 (segment (start 3.898531 -16.166741) (end 4.240895 -16.509105) (width 0.25) (layer "F.Cu") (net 3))
 (segment (start 13 -19.1) (end 13.15 -19.25) (width 0.25) (layer "F.Cu") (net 3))
 (segment (start 3.898531 -11.5137) (end 3.898531 -16.166741) (width 0.25) (layer "F.Cu") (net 3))
 (segment (start 5.73179 -18) (end 13 -18) (width 0.25) (layer "F.Cu") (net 3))
 (segment (start 3.501 -11.116168) (end 3.898531 -11.5137) (width 0.25) (layer "F.Cu") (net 3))
 (segment (start 4.240895 -16.509105) (end 5.73179 -18) (width 0.25) (layer "F.Cu") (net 3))
 (segment (start 3.501 -3.396) (end 3.501 -11.116168) (width 0.25) (layer "F.Cu") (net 3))
 (segment (start 3.449011 -11.699897) (end 3.449011 -12.300989) (width 0.25) (layer "F.Cu") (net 10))
 (segment (start 3 -12.75) (end 3 -15.903928) (width 0.25) (layer "F.Cu") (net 10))
 (segment (start 5.9 -18.803928) (end 5.9 -19.25) (width 0.25) (layer "F.Cu") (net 10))
 (segment (start 3.001 -11.251886) (end 3.449011 -11.699897) (width 0.25) (layer "F.Cu") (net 10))
 (segment (start 3.001 -3.396) (end 3.001 -11.251886) (width 0.25) (layer "F.Cu") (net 10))
 (segment (start 3.449011 -12.300989) (end 3 -12.75) (width 0.25) (layer "F.Cu") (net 10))
 (segment (start 3 -15.903928) (end 5.9 -18.803928) (width 0.25) (layer "F.Cu") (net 10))
 (segment (start 2 -15.903928) (end 4.9 -18.803928) (width 0.25) (layer "F.Cu") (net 11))
 (segment (start 2 -3.396) (end 2 -15.903928) (width 0.25) (layer "F.Cu") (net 11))
 (segment (start 4.9 -18.803928) (end 4.9 -19.25) (width 0.25) (layer "F.Cu") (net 11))
 (segment (start 1.5 -3.396) (end 1.5 -9.75) (width 0.25) (layer "F.Cu") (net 7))
 (segment (start -2.5 -13.75) (end -2.5 -19) (width 0.25) (layer "F.Cu") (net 7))
 (segment (start -2.5 -19) (end -2.25 -19.25) (width 0.25) (layer "F.Cu") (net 7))
 (segment (start 1.5 -9.75) (end -2.5 -13.75) (width 0.25) (layer "F.Cu") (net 7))
 (segment (start 0.5 -8.611733) (end -4.25 -13.361733) (width 0.25) (layer "F.Cu") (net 8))
 (segment (start -4.25 -13.361733) (end -4.25 -14) (width 0.25) (layer "F.Cu") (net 8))
 (segment (start -4.25 -14) (end -4.25 -19.25) (width 0.25) (layer "F.Cu") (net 8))
 (segment (start 0.5 -3.396) (end 0.5 -8.611733) (width 0.25) (layer "F.Cu") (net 8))
 (segment (start -10.95 -18.350424) (end -10.95 -19.25) (width 0.25) (layer "F.Cu") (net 5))
 (segment (start 0 -8.476016) (end -2.599196 -11.075212) (width 0.25) (layer "F.Cu") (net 5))
 (segment (start -2.599196 -11.075212) (end -3.674788 -11.075212) (width 0.25) (layer "F.Cu") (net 5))
 (segment (start -3.674788 -11.075212) (end -10.95 -18.350424) (width 0.25) (layer "F.Cu") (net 5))
 (segment (start 0 -3.396) (end 0 -8.476016) (width 0.25) (layer "F.Cu") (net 5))
 (segment (start -12.823196 -19.25) (end -12.95 -19.25) (width 0.25) (layer "F.Cu") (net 6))
 (segment (start -1 -3.396) (end -1 -7.426804) (width 0.25) (layer "F.Cu") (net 6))
 (segment (start -1 -7.426804) (end -12.823196 -19.25) (width 0.25) (layer "F.Cu") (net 6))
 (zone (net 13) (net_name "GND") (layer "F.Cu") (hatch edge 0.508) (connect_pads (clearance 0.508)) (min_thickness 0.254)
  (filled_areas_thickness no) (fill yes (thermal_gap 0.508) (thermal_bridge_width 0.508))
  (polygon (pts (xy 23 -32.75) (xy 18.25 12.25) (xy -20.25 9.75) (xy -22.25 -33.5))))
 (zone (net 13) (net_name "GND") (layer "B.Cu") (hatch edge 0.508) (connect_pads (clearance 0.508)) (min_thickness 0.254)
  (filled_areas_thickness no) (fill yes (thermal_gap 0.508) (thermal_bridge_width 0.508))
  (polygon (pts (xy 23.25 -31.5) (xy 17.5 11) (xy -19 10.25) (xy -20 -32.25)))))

